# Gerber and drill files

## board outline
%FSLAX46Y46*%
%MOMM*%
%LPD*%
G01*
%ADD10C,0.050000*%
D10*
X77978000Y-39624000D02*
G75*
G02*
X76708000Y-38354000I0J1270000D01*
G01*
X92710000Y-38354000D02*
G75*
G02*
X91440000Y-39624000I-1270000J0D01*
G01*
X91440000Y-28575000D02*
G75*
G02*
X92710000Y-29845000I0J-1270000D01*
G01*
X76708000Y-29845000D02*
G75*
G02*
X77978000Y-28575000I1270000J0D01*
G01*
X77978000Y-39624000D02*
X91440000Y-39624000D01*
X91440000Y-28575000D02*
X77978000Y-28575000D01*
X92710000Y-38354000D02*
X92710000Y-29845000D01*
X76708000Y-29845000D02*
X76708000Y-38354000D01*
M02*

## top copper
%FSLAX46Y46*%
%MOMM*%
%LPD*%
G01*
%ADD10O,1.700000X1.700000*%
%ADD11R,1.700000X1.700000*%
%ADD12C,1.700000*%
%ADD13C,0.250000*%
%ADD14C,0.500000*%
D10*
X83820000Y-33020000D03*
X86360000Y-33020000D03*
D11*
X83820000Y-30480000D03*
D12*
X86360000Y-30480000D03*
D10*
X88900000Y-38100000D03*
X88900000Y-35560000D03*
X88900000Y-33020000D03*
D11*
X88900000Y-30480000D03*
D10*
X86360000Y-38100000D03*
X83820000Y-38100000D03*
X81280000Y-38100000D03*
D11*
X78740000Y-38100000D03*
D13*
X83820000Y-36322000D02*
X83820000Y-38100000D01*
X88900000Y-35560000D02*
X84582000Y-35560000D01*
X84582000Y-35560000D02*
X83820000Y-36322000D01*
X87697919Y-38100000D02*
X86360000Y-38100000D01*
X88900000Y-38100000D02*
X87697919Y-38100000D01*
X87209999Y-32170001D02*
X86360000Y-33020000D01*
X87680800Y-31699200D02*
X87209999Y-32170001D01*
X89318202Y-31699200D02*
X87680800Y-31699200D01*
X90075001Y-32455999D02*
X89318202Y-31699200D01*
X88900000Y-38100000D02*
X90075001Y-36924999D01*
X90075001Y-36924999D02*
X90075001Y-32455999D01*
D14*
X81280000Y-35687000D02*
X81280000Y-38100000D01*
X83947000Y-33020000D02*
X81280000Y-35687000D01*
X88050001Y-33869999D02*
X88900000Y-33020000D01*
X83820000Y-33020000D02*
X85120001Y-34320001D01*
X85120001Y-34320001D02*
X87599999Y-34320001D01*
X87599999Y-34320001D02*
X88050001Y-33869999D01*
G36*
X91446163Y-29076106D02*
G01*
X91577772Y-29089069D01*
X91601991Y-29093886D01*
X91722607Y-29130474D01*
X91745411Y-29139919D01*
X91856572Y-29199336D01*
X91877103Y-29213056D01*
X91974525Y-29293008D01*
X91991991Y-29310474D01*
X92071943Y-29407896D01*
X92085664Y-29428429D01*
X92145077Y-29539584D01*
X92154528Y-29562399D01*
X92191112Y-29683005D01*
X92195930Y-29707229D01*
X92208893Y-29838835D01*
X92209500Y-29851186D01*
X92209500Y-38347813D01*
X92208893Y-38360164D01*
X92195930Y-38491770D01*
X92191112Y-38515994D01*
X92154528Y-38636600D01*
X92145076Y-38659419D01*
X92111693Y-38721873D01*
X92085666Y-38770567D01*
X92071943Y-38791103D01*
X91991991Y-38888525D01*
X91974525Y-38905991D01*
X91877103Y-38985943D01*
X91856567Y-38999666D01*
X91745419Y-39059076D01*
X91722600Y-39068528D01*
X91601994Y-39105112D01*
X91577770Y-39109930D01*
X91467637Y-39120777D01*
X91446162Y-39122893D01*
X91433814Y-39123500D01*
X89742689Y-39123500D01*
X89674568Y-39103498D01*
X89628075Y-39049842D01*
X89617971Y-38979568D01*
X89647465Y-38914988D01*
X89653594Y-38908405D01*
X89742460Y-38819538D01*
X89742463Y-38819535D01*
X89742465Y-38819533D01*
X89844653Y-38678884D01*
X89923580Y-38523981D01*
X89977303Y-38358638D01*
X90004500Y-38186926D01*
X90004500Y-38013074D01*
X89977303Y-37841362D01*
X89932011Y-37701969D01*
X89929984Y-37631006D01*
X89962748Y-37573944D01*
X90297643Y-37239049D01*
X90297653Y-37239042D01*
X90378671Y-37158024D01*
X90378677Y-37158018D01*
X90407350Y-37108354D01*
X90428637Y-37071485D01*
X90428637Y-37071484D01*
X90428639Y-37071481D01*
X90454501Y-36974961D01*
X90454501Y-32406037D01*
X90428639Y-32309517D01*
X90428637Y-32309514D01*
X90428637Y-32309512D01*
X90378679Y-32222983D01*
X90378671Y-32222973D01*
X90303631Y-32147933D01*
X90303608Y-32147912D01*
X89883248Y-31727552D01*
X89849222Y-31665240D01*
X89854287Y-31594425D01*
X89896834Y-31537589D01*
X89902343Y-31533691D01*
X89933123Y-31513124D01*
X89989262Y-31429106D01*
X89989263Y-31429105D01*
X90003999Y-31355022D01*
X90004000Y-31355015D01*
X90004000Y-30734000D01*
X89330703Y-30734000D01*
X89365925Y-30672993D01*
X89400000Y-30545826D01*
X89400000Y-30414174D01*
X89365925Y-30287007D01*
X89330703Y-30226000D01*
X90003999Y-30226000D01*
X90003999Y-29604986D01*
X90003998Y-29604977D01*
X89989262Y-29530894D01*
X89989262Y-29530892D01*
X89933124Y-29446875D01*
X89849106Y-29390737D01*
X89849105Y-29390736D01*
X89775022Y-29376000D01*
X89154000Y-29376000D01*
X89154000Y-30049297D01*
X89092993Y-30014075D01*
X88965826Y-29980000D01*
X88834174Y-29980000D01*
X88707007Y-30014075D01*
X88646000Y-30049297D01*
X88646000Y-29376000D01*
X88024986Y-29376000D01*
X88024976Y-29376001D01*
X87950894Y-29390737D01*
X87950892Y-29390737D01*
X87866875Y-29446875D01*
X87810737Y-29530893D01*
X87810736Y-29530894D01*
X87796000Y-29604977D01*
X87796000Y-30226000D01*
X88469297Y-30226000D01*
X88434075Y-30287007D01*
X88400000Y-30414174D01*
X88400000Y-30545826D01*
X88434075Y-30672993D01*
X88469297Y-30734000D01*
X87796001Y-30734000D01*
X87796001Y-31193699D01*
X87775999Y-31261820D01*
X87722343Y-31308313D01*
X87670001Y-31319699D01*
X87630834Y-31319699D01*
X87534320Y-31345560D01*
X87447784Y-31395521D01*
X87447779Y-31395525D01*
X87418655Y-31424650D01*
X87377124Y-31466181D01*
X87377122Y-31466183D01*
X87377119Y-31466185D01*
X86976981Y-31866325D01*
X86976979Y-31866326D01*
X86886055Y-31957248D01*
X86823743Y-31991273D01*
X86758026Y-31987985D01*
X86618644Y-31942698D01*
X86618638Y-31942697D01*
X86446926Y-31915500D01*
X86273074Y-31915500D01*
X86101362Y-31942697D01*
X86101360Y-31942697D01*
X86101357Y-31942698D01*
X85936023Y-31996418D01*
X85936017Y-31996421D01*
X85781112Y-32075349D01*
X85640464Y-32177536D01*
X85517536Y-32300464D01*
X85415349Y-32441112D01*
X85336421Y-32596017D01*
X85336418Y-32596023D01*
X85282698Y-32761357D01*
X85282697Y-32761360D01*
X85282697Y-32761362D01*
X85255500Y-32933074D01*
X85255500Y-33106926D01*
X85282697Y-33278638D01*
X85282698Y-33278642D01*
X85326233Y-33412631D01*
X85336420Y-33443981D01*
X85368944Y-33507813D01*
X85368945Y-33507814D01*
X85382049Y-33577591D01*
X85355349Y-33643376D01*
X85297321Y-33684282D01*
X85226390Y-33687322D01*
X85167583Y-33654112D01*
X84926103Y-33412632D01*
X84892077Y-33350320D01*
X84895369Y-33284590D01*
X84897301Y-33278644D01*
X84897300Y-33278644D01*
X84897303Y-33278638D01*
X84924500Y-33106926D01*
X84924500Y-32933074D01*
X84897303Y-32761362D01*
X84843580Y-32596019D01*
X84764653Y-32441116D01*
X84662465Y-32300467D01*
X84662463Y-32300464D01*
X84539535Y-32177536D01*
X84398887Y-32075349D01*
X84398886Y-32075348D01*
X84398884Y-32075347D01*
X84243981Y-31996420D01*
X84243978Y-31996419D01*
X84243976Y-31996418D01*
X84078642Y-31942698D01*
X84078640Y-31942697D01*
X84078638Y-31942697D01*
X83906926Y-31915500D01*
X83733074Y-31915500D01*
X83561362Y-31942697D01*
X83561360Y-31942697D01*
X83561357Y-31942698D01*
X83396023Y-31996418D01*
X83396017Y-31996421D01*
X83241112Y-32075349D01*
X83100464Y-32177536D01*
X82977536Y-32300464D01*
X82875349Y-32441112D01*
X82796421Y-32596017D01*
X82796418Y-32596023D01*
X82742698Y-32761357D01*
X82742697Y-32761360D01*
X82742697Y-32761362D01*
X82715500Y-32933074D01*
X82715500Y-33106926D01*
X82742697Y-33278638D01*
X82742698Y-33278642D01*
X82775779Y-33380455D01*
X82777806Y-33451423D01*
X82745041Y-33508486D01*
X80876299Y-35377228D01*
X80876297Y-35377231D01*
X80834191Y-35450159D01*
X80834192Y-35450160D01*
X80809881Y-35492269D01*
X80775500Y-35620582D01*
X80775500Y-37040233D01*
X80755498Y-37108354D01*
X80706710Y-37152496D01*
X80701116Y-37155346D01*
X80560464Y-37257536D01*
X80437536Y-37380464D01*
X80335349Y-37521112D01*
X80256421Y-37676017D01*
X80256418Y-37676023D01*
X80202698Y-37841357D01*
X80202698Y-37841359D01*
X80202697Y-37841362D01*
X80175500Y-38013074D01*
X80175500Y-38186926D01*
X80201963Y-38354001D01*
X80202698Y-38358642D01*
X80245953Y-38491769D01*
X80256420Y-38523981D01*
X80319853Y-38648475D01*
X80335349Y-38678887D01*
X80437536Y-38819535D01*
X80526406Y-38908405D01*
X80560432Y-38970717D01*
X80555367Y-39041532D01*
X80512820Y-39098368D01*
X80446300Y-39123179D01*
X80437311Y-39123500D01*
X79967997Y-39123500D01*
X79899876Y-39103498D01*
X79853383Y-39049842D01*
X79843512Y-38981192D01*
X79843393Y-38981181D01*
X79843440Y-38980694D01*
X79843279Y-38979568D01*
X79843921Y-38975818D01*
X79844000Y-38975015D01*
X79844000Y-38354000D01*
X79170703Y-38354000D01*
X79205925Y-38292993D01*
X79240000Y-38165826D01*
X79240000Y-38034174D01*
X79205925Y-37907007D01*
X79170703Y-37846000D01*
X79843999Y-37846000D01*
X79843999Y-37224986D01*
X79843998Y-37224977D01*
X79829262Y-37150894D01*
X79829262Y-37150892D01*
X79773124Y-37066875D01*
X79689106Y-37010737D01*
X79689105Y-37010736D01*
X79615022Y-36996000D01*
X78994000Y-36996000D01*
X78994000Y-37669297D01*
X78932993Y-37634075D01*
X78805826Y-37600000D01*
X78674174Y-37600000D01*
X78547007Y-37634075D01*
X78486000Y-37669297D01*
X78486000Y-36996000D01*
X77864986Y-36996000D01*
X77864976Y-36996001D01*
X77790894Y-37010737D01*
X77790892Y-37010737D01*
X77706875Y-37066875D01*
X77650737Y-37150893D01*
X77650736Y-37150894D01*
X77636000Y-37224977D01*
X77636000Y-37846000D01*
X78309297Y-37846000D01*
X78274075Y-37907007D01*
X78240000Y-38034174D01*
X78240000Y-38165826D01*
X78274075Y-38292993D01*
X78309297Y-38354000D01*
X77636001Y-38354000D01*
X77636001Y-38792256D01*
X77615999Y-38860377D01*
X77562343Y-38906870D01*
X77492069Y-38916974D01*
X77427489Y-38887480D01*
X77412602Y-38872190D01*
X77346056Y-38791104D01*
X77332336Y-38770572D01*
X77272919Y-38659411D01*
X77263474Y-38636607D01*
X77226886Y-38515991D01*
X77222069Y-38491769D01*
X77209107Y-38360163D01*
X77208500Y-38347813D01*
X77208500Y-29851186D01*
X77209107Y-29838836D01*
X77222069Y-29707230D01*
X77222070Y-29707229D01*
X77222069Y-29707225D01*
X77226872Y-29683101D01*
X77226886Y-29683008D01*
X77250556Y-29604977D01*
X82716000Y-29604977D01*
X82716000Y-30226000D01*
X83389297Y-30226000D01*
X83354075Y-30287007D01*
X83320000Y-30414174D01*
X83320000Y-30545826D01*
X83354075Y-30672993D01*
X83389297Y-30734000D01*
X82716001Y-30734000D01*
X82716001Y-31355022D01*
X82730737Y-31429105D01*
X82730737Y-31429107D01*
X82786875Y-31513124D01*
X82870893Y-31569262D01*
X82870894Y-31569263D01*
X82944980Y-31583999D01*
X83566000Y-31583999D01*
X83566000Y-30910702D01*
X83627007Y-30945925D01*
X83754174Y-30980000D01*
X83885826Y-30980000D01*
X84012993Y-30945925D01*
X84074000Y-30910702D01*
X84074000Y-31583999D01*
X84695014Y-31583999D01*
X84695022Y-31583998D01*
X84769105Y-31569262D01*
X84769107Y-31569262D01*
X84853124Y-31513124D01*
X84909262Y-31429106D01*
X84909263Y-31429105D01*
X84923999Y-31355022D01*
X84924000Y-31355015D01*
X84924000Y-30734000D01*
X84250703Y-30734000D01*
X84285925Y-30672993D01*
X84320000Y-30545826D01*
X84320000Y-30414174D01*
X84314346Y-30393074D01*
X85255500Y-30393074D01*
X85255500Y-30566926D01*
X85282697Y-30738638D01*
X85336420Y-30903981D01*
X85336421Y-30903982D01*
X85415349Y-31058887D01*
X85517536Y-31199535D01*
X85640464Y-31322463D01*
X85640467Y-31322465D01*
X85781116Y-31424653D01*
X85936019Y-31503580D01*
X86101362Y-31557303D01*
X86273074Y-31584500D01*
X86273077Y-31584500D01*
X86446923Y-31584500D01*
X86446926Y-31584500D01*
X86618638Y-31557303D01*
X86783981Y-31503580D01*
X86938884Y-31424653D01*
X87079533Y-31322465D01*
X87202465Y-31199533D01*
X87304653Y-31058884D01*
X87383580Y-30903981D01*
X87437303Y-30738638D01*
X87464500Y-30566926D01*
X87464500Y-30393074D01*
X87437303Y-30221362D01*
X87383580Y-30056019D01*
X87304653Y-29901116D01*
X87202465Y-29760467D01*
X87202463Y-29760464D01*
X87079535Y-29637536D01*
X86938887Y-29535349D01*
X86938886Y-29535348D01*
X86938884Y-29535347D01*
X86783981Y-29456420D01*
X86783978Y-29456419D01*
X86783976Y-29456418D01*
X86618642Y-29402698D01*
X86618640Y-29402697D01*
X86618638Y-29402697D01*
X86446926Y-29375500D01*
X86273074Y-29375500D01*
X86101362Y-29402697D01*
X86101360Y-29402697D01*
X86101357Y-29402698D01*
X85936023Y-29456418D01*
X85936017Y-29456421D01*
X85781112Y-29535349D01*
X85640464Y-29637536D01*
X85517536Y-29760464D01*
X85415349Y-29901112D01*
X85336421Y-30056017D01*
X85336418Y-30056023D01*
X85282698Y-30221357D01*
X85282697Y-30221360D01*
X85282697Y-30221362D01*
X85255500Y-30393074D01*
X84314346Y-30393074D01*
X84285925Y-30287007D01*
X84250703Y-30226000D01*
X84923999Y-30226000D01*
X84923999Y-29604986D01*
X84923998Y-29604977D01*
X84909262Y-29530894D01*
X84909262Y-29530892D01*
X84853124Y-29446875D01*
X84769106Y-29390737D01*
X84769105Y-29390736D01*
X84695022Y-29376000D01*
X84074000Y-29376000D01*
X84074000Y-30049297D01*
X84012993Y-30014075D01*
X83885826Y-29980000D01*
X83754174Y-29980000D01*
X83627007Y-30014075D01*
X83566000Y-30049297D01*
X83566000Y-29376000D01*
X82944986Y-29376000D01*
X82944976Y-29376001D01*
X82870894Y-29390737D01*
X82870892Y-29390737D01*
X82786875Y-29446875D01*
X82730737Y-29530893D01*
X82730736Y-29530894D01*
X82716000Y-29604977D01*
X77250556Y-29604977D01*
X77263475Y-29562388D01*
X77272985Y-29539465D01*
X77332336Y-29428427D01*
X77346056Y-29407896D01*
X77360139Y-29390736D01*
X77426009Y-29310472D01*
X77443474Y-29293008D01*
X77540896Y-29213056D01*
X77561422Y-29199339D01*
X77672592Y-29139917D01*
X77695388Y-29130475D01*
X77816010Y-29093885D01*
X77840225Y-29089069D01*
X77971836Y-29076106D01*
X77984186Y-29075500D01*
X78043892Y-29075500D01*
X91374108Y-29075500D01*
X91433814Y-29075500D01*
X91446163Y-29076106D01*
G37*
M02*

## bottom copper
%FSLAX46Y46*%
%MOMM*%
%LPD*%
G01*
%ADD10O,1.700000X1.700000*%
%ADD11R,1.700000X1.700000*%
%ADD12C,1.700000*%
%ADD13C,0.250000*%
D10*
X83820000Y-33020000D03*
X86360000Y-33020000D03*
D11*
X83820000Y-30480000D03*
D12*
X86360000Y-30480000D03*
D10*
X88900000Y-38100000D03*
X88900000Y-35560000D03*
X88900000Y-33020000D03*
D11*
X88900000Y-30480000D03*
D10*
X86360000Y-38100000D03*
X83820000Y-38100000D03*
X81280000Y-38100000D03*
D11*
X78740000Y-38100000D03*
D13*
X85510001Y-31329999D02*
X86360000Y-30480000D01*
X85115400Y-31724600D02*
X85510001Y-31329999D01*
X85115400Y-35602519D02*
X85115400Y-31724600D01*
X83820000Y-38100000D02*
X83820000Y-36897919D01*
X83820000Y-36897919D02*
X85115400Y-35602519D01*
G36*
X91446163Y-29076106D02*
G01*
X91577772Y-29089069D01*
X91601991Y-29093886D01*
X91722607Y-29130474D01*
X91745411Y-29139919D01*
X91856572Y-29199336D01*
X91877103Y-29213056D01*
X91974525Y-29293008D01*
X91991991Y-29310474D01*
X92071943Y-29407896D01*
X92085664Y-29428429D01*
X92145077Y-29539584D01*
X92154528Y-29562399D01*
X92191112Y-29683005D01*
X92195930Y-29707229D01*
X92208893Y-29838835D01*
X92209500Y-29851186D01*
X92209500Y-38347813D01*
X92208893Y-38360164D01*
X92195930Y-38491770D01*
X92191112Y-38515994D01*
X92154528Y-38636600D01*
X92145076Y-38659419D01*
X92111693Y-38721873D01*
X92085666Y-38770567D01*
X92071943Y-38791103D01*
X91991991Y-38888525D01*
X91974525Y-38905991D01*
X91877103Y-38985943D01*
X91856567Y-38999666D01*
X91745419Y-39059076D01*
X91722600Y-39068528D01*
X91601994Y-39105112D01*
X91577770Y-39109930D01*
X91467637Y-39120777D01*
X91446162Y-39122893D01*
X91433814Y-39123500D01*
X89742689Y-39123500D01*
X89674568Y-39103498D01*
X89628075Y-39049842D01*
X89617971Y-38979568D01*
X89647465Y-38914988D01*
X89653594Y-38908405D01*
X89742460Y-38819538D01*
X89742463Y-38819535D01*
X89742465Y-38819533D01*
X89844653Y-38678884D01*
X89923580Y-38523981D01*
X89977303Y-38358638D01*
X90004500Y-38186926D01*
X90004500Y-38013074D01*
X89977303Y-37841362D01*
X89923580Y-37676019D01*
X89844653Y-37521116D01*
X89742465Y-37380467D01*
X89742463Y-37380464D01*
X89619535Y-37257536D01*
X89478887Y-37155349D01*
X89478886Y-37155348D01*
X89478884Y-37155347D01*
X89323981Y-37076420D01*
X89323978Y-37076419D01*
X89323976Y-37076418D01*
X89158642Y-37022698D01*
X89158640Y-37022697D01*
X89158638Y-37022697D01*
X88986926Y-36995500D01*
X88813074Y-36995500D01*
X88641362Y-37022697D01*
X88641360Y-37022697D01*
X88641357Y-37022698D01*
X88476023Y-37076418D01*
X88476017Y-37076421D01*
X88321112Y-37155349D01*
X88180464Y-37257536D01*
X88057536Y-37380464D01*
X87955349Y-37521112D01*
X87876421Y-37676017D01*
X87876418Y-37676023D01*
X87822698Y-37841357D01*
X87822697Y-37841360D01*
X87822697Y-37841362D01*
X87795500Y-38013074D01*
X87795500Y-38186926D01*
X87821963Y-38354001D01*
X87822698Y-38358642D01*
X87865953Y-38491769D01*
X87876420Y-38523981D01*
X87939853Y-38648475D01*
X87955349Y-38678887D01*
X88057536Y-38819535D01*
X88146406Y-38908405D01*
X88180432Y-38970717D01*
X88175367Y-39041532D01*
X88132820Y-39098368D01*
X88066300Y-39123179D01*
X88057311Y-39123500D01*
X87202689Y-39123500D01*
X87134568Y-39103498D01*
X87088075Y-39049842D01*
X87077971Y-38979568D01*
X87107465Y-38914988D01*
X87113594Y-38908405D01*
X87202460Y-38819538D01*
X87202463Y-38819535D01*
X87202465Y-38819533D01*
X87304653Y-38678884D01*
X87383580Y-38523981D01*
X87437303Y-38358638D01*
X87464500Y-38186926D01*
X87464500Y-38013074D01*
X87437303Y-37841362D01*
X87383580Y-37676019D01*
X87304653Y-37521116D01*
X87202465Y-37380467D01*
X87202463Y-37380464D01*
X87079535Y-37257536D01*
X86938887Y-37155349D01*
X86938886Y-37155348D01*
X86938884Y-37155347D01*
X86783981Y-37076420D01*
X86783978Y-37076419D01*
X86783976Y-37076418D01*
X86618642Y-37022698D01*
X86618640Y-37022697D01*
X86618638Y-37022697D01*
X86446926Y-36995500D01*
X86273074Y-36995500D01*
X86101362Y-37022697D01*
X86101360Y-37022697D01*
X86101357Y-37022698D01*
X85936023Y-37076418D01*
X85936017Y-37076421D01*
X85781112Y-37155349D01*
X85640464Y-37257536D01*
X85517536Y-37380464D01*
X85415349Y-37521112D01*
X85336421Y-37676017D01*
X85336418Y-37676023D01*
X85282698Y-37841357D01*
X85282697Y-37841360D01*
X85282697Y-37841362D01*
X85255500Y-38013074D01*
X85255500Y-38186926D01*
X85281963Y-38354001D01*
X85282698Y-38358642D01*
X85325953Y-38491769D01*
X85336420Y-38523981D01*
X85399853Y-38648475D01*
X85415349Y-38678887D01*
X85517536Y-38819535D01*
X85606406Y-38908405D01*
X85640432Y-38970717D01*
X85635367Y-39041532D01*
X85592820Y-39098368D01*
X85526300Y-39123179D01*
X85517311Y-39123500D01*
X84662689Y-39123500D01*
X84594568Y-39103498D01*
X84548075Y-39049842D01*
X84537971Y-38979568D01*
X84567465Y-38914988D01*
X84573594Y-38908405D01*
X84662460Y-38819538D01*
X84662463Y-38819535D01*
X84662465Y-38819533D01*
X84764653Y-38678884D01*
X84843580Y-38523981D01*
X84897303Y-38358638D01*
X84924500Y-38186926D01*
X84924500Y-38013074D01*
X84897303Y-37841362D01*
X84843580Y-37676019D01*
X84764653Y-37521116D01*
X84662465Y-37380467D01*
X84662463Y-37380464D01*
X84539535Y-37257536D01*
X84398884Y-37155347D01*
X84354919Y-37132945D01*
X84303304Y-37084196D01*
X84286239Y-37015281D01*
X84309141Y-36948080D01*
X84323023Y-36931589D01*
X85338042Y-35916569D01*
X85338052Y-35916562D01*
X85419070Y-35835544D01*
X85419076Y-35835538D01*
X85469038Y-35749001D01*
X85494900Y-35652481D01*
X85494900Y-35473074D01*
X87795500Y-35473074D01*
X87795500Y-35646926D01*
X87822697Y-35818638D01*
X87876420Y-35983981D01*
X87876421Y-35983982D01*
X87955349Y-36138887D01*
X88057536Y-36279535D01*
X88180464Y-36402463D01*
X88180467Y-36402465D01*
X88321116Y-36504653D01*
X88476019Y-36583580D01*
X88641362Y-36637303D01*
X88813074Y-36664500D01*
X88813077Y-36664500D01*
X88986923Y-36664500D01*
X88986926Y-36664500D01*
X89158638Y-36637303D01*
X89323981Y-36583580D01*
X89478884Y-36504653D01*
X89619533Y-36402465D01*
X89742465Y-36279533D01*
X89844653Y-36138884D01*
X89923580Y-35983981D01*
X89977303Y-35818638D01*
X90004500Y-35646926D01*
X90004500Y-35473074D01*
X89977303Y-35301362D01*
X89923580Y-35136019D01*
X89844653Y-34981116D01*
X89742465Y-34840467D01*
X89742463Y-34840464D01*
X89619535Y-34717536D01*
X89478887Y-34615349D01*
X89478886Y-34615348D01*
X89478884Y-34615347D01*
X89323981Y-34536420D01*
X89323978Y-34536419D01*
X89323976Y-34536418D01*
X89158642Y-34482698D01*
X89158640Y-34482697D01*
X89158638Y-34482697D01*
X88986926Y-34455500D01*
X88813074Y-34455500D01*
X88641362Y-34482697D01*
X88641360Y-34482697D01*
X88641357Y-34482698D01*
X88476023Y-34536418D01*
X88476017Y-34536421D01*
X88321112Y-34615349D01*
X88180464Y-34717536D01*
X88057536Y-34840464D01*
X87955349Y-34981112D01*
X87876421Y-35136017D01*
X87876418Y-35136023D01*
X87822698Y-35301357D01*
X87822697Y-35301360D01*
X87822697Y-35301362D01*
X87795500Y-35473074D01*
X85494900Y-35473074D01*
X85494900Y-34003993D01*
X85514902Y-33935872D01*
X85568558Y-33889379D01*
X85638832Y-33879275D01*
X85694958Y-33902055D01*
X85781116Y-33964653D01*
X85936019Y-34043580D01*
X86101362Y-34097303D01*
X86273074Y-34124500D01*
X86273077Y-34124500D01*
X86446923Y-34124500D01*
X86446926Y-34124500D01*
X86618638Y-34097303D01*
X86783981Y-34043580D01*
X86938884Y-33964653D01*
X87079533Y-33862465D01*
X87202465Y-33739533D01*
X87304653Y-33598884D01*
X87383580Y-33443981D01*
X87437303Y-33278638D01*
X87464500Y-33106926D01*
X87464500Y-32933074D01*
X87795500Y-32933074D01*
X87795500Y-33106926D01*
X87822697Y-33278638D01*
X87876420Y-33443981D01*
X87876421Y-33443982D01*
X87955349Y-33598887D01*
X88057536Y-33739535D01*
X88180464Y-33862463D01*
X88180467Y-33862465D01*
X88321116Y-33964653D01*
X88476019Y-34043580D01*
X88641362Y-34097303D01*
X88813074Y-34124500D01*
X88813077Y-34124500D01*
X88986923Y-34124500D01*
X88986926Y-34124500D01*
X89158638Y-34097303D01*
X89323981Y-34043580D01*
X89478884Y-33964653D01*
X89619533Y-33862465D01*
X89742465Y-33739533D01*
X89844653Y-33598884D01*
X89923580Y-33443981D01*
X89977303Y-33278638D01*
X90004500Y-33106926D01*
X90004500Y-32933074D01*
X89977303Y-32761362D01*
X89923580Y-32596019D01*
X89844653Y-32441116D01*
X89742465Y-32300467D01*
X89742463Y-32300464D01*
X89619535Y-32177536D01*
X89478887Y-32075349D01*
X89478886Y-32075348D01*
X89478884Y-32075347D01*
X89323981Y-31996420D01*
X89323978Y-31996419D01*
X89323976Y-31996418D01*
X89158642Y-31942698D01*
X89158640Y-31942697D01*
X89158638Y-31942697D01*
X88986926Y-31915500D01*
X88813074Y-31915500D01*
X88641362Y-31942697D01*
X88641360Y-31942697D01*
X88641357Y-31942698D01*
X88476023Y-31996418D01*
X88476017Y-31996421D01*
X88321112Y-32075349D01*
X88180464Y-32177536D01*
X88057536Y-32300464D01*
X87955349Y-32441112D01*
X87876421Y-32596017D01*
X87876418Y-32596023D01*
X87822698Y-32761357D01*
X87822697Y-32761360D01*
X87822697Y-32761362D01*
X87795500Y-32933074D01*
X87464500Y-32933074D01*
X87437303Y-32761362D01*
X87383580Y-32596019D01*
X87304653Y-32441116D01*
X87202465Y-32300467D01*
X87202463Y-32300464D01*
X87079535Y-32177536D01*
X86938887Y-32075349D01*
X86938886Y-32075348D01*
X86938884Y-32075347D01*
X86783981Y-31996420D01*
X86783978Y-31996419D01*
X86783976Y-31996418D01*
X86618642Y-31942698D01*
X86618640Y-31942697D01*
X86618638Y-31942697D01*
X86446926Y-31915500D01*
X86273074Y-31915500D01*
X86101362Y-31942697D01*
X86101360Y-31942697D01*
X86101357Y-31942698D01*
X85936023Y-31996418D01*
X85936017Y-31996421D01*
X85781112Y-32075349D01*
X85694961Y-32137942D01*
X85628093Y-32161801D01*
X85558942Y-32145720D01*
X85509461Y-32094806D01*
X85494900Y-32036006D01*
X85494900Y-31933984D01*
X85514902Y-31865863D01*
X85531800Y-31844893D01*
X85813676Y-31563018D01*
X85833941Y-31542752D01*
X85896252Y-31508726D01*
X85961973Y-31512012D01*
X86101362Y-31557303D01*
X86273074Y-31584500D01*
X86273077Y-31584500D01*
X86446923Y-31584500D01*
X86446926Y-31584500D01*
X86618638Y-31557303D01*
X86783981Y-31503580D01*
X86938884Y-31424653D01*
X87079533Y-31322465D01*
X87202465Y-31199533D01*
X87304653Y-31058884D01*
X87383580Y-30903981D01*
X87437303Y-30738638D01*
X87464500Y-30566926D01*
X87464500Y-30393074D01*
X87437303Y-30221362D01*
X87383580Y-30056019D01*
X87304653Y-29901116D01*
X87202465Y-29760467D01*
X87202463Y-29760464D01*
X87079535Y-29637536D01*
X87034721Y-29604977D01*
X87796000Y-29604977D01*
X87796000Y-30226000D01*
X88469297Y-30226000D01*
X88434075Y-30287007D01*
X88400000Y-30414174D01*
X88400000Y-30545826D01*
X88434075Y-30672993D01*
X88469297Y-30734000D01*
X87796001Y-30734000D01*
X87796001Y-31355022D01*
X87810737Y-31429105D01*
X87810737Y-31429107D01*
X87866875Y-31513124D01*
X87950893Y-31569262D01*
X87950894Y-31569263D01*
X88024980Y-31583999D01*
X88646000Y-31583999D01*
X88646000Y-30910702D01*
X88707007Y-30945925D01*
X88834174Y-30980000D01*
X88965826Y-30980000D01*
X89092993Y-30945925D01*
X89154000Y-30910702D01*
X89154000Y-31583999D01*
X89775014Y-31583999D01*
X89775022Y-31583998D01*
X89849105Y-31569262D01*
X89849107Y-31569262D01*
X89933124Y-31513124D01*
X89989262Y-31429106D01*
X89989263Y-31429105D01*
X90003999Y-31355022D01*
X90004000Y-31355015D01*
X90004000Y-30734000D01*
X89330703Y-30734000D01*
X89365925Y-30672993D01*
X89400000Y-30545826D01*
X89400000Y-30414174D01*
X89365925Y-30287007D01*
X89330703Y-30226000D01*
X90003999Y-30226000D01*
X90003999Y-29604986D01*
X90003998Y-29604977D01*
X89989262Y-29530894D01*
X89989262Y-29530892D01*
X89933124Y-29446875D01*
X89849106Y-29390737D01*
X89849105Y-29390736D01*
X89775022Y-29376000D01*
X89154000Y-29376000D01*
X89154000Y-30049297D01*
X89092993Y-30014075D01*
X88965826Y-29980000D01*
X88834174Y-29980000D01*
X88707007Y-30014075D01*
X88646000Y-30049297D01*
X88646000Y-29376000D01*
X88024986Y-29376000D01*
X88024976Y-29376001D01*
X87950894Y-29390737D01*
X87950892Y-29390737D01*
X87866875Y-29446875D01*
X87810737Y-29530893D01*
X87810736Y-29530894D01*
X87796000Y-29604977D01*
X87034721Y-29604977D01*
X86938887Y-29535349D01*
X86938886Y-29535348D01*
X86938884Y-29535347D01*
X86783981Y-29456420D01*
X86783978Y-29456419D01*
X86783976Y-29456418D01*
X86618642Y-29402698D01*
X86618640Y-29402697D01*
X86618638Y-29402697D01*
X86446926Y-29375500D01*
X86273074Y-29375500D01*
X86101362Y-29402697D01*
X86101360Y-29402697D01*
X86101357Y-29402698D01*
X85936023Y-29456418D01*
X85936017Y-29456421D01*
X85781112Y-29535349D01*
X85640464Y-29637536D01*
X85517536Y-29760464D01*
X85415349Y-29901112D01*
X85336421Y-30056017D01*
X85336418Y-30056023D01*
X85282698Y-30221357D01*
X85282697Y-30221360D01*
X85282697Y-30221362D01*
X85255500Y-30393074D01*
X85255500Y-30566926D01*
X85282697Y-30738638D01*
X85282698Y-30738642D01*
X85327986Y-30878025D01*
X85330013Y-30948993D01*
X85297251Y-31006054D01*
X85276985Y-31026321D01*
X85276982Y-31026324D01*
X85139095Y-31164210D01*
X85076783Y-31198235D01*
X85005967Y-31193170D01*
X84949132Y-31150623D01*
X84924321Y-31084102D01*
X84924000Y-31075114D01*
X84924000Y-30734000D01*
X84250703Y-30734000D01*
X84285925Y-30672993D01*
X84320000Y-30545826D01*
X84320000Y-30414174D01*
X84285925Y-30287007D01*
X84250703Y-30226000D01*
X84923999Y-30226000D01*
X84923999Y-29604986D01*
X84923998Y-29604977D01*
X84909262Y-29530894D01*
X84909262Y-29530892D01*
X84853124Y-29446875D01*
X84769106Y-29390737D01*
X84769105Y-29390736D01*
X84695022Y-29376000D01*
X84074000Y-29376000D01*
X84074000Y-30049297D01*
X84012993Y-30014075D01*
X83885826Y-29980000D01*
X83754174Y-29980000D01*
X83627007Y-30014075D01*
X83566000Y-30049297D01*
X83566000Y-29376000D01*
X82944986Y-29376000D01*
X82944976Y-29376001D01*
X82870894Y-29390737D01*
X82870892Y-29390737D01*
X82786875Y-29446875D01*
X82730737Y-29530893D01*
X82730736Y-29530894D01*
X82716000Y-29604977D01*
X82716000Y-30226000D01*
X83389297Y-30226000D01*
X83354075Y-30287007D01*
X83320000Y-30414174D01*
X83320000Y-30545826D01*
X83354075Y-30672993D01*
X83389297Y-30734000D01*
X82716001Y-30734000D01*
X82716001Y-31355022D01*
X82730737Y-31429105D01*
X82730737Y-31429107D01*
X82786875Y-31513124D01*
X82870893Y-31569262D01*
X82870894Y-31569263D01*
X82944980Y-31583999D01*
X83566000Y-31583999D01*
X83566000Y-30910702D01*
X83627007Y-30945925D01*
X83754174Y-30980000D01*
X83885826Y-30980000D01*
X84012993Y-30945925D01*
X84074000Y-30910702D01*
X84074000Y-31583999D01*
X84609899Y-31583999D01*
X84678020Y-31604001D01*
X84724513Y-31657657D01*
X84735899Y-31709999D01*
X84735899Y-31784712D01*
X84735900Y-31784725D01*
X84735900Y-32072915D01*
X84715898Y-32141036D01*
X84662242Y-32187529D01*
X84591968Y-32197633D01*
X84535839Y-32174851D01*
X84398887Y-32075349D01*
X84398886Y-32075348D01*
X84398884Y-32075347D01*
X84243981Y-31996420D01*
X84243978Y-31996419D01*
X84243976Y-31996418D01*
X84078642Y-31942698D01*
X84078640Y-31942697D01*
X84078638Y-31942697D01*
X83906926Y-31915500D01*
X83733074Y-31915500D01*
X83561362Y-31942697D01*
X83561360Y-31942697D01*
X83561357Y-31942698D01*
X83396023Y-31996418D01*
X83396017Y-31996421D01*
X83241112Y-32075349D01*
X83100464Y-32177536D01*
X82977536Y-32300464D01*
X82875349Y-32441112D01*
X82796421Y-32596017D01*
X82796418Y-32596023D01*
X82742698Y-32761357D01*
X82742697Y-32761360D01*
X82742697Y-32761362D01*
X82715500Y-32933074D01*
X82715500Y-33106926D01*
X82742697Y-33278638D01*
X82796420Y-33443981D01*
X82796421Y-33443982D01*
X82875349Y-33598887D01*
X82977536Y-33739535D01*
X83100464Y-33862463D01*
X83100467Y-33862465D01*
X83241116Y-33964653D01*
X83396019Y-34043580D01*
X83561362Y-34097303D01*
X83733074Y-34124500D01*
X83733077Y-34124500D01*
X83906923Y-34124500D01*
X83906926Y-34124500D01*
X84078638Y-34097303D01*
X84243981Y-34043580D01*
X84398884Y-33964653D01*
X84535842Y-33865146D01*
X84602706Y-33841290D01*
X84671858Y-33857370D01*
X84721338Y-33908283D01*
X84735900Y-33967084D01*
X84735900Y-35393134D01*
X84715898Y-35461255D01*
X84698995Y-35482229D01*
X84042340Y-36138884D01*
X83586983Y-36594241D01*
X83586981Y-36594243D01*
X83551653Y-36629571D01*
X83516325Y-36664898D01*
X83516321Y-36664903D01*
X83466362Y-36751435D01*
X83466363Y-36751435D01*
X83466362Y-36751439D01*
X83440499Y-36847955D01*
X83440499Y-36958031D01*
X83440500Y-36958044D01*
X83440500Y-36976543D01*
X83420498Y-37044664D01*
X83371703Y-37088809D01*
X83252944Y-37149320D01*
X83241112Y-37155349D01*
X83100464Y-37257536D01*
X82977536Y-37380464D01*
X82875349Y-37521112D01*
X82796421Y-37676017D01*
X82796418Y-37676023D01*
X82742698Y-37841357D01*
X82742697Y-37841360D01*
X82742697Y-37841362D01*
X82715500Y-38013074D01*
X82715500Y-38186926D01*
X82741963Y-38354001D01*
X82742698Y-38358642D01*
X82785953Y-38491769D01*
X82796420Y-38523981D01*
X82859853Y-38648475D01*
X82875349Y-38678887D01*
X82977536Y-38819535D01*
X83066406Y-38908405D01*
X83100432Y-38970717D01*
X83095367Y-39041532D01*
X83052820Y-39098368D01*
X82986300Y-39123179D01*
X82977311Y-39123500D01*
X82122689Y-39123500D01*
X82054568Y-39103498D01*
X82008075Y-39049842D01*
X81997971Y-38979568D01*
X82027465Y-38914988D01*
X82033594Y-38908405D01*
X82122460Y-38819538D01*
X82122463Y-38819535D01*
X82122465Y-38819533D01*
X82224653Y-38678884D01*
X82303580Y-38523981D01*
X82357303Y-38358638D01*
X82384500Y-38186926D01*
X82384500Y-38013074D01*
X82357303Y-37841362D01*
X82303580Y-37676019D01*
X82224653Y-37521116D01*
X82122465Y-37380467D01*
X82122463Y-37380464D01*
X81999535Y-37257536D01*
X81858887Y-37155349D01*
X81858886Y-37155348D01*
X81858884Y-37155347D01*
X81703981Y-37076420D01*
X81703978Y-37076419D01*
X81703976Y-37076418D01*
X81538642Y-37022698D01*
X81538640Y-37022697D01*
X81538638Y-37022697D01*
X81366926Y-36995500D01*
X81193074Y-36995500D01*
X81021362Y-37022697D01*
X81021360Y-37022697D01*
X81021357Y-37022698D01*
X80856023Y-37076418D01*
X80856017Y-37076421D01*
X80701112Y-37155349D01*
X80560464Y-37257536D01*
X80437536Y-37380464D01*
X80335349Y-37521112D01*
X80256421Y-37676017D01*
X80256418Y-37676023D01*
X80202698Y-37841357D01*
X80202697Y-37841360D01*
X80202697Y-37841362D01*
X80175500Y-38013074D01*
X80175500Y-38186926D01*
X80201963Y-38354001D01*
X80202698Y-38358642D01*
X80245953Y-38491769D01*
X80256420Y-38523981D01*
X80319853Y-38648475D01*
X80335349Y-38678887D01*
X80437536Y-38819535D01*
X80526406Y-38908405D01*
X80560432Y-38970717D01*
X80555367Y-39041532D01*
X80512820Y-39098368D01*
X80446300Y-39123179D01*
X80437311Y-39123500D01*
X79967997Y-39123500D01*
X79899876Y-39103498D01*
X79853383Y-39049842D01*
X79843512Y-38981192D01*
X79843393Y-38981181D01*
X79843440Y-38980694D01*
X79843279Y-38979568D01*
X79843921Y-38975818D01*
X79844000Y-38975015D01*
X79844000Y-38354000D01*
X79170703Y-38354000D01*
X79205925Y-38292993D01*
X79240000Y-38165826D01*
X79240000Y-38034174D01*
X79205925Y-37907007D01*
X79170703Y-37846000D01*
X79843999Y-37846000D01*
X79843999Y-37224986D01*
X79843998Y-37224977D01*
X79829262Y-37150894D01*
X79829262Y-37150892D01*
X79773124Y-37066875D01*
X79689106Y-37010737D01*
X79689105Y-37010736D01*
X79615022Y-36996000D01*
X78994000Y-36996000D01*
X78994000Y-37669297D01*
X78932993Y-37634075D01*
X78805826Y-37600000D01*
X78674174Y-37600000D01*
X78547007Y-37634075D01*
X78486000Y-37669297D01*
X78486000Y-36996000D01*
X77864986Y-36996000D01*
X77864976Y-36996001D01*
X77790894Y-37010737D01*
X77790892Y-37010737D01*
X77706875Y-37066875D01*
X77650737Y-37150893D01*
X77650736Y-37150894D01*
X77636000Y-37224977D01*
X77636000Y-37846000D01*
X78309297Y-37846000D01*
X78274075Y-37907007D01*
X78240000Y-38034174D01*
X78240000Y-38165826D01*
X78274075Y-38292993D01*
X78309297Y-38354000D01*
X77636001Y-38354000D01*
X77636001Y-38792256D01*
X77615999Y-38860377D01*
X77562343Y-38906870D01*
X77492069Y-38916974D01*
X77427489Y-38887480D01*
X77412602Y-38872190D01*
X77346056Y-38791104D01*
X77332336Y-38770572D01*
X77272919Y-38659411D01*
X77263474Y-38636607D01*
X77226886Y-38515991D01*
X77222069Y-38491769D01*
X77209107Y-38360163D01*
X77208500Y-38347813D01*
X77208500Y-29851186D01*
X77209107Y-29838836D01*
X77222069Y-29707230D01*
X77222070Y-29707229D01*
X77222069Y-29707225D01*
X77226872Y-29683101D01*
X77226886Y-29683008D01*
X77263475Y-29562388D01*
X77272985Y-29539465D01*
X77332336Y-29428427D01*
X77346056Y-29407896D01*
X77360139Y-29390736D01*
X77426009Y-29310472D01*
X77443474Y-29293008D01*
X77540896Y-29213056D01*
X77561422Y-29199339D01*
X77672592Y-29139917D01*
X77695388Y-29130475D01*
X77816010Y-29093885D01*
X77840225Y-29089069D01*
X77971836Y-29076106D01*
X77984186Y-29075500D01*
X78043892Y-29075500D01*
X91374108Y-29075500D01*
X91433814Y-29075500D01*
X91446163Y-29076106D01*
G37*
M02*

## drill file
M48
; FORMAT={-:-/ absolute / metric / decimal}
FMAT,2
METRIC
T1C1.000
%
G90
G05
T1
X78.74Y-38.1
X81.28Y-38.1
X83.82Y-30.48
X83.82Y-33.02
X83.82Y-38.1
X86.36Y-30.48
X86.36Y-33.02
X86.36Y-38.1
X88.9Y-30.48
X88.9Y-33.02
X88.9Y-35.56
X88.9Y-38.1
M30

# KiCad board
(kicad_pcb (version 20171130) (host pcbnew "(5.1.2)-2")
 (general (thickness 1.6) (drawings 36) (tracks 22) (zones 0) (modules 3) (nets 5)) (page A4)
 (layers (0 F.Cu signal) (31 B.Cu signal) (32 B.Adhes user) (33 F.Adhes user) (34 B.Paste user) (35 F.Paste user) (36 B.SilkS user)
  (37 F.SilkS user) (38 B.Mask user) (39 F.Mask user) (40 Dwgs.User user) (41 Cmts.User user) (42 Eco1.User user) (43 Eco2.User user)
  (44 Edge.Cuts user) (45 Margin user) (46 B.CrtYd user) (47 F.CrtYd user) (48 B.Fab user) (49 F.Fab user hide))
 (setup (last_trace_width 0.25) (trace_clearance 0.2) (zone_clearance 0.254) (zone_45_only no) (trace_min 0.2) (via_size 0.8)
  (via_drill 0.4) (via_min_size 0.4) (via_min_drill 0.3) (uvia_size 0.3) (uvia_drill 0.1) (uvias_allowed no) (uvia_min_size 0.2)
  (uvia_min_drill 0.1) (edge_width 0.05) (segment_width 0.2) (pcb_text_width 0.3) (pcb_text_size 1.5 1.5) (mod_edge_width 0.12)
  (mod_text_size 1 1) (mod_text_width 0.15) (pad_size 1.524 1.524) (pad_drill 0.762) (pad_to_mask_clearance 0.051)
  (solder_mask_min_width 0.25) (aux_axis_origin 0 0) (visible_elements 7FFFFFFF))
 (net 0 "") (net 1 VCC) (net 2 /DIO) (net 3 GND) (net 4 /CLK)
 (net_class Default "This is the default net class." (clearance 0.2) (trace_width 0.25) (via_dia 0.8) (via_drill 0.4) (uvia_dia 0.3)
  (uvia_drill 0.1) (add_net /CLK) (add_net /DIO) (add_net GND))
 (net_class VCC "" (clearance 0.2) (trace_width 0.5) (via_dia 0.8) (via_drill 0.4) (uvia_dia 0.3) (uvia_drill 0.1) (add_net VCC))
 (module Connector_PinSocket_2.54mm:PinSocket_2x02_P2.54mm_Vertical (layer F.Cu) (at 83.82 30.48)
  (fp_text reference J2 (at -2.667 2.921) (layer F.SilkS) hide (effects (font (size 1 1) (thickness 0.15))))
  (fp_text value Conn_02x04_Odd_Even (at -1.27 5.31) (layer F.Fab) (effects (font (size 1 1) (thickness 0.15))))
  (pad 2 thru_hole oval (at 0 2.54) (size 1.7 1.7) (drill 1) (layers *.Cu *.Mask) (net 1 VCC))
  (pad 4 thru_hole oval (at 2.54 2.54) (size 1.7 1.7) (drill 1) (layers *.Cu *.Mask) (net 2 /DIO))
  (pad 1 thru_hole rect (at 0 0) (size 1.7 1.7) (drill 1) (layers *.Cu *.Mask) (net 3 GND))
  (pad 3 thru_hole circle (at 2.54 0) (size 1.7 1.7) (drill 1) (layers *.Cu *.Mask) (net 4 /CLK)))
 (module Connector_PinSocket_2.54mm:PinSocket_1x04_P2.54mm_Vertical (layer F.Cu) (at 88.9 30.48)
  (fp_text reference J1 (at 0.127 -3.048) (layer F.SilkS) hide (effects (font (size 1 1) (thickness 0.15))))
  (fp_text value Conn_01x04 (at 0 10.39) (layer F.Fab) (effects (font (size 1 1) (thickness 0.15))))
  (pad 4 thru_hole oval (at 0 7.62) (size 1.7 1.7) (drill 1) (layers *.Cu *.Mask) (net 2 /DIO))
  (pad 3 thru_hole oval (at 0 5.08) (size 1.7 1.7) (drill 1) (layers *.Cu *.Mask) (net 4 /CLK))
  (pad 2 thru_hole oval (at 0 2.54) (size 1.7 1.7) (drill 1) (layers *.Cu *.Mask) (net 1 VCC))
  (pad 1 thru_hole rect (at 0 0) (size 1.7 1.7) (drill 1) (layers *.Cu *.Mask) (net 3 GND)))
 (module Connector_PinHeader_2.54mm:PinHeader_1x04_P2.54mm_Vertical (layer F.Cu) (at 78.74 38.1 90)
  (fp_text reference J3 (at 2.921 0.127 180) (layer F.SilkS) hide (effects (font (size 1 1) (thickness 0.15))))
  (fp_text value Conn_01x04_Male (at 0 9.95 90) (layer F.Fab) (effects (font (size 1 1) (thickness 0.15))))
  (pad 4 thru_hole oval (at 0 7.62 90) (size 1.7 1.7) (drill 1) (layers *.Cu *.Mask) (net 2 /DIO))
  (pad 3 thru_hole oval (at 0 5.08 90) (size 1.7 1.7) (drill 1) (layers *.Cu *.Mask) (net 4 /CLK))
  (pad 2 thru_hole oval (at 0 2.54 90) (size 1.7 1.7) (drill 1) (layers *.Cu *.Mask) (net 1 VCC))
  (pad 1 thru_hole rect (at 0 0 90) (size 1.7 1.7) (drill 1) (layers *.Cu *.Mask) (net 3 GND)))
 (gr_arc (start 77.978 38.354) (end 76.708 38.354) (angle -90) (layer Edge.Cuts) (width 0.05))
 (gr_arc (start 91.44 38.354) (end 91.44 39.624) (angle -90) (layer Edge.Cuts) (width 0.05))
 (gr_arc (start 91.44 29.845) (end 92.71 29.845) (angle -90) (layer Edge.Cuts) (width 0.05))
 (gr_arc (start 77.978 29.845) (end 77.978 28.575) (angle -90) (layer Edge.Cuts) (width 0.05))
 (gr_line (start 77.978 39.624) (end 91.44 39.624) (layer Edge.Cuts) (width 0.05))
 (gr_line (start 91.44 28.575) (end 77.978 28.575) (layer Edge.Cuts) (width 0.05))
 (gr_line (start 92.71 38.354) (end 92.71 29.845) (layer Edge.Cuts) (width 0.05))
 (gr_line (start 76.708 29.845) (end 76.708 38.354) (layer Edge.Cuts) (width 0.05))
 (segment (start 83.82 36.322) (end 83.82 38.1) (width 0.25) (layer F.Cu) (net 4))
 (segment (start 88.9 35.56) (end 84.582 35.56) (width 0.25) (layer F.Cu) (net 4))
 (segment (start 84.582 35.56) (end 83.82 36.322) (width 0.25) (layer F.Cu) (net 4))
 (segment (start 85.510001 31.329999) (end 86.36 30.48) (width 0.25) (layer B.Cu) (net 4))
 (segment (start 85.1154 31.7246) (end 85.510001 31.329999) (width 0.25) (layer B.Cu) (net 4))
 (segment (start 85.1154 35.602519) (end 85.1154 31.7246) (width 0.25) (layer B.Cu) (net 4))
 (segment (start 83.82 38.1) (end 83.82 36.897919) (width 0.25) (layer B.Cu) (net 4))
 (segment (start 83.82 36.897919) (end 85.1154 35.602519) (width 0.25) (layer B.Cu) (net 4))
 (segment (start 87.697919 38.1) (end 86.36 38.1) (width 0.25) (layer F.Cu) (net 2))
 (segment (start 88.9 38.1) (end 87.697919 38.1) (width 0.25) (layer F.Cu) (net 2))
 (segment (start 87.209999 32.170001) (end 86.36 33.02) (width 0.25) (layer F.Cu) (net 2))
 (segment (start 87.6808 31.6992) (end 87.209999 32.170001) (width 0.25) (layer F.Cu) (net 2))
 (segment (start 89.318202 31.6992) (end 87.6808 31.6992) (width 0.25) (layer F.Cu) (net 2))
 (segment (start 90.075001 32.455999) (end 89.318202 31.6992) (width 0.25) (layer F.Cu) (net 2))
 (segment (start 88.9 38.1) (end 90.075001 36.924999) (width 0.25) (layer F.Cu) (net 2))
 (segment (start 90.075001 36.924999) (end 90.075001 32.455999) (width 0.25) (layer F.Cu) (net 2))
 (segment (start 81.28 35.687) (end 81.28 38.1) (width 0.5) (layer F.Cu) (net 1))
 (segment (start 83.947 33.02) (end 81.28 35.687) (width 0.5) (layer F.Cu) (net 1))
 (segment (start 88.050001 33.869999) (end 88.9 33.02) (width 0.5) (layer F.Cu) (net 1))
 (segment (start 83.82 33.02) (end 85.120001 34.320001) (width 0.5) (layer F.Cu) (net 1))
 (segment (start 85.120001 34.320001) (end 87.599999 34.320001) (width 0.5) (layer F.Cu) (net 1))
 (segment (start 87.599999 34.320001) (end 88.050001 33.869999) (width 0.5) (layer F.Cu) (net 1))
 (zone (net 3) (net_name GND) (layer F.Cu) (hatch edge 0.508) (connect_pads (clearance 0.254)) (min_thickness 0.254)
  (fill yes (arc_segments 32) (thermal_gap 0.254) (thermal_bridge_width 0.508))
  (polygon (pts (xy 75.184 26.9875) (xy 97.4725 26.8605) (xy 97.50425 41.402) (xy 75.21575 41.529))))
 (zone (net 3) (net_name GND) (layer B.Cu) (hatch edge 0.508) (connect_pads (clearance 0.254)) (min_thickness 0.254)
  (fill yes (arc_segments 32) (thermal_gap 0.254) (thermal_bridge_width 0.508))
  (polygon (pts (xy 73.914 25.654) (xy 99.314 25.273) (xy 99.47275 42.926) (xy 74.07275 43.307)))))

